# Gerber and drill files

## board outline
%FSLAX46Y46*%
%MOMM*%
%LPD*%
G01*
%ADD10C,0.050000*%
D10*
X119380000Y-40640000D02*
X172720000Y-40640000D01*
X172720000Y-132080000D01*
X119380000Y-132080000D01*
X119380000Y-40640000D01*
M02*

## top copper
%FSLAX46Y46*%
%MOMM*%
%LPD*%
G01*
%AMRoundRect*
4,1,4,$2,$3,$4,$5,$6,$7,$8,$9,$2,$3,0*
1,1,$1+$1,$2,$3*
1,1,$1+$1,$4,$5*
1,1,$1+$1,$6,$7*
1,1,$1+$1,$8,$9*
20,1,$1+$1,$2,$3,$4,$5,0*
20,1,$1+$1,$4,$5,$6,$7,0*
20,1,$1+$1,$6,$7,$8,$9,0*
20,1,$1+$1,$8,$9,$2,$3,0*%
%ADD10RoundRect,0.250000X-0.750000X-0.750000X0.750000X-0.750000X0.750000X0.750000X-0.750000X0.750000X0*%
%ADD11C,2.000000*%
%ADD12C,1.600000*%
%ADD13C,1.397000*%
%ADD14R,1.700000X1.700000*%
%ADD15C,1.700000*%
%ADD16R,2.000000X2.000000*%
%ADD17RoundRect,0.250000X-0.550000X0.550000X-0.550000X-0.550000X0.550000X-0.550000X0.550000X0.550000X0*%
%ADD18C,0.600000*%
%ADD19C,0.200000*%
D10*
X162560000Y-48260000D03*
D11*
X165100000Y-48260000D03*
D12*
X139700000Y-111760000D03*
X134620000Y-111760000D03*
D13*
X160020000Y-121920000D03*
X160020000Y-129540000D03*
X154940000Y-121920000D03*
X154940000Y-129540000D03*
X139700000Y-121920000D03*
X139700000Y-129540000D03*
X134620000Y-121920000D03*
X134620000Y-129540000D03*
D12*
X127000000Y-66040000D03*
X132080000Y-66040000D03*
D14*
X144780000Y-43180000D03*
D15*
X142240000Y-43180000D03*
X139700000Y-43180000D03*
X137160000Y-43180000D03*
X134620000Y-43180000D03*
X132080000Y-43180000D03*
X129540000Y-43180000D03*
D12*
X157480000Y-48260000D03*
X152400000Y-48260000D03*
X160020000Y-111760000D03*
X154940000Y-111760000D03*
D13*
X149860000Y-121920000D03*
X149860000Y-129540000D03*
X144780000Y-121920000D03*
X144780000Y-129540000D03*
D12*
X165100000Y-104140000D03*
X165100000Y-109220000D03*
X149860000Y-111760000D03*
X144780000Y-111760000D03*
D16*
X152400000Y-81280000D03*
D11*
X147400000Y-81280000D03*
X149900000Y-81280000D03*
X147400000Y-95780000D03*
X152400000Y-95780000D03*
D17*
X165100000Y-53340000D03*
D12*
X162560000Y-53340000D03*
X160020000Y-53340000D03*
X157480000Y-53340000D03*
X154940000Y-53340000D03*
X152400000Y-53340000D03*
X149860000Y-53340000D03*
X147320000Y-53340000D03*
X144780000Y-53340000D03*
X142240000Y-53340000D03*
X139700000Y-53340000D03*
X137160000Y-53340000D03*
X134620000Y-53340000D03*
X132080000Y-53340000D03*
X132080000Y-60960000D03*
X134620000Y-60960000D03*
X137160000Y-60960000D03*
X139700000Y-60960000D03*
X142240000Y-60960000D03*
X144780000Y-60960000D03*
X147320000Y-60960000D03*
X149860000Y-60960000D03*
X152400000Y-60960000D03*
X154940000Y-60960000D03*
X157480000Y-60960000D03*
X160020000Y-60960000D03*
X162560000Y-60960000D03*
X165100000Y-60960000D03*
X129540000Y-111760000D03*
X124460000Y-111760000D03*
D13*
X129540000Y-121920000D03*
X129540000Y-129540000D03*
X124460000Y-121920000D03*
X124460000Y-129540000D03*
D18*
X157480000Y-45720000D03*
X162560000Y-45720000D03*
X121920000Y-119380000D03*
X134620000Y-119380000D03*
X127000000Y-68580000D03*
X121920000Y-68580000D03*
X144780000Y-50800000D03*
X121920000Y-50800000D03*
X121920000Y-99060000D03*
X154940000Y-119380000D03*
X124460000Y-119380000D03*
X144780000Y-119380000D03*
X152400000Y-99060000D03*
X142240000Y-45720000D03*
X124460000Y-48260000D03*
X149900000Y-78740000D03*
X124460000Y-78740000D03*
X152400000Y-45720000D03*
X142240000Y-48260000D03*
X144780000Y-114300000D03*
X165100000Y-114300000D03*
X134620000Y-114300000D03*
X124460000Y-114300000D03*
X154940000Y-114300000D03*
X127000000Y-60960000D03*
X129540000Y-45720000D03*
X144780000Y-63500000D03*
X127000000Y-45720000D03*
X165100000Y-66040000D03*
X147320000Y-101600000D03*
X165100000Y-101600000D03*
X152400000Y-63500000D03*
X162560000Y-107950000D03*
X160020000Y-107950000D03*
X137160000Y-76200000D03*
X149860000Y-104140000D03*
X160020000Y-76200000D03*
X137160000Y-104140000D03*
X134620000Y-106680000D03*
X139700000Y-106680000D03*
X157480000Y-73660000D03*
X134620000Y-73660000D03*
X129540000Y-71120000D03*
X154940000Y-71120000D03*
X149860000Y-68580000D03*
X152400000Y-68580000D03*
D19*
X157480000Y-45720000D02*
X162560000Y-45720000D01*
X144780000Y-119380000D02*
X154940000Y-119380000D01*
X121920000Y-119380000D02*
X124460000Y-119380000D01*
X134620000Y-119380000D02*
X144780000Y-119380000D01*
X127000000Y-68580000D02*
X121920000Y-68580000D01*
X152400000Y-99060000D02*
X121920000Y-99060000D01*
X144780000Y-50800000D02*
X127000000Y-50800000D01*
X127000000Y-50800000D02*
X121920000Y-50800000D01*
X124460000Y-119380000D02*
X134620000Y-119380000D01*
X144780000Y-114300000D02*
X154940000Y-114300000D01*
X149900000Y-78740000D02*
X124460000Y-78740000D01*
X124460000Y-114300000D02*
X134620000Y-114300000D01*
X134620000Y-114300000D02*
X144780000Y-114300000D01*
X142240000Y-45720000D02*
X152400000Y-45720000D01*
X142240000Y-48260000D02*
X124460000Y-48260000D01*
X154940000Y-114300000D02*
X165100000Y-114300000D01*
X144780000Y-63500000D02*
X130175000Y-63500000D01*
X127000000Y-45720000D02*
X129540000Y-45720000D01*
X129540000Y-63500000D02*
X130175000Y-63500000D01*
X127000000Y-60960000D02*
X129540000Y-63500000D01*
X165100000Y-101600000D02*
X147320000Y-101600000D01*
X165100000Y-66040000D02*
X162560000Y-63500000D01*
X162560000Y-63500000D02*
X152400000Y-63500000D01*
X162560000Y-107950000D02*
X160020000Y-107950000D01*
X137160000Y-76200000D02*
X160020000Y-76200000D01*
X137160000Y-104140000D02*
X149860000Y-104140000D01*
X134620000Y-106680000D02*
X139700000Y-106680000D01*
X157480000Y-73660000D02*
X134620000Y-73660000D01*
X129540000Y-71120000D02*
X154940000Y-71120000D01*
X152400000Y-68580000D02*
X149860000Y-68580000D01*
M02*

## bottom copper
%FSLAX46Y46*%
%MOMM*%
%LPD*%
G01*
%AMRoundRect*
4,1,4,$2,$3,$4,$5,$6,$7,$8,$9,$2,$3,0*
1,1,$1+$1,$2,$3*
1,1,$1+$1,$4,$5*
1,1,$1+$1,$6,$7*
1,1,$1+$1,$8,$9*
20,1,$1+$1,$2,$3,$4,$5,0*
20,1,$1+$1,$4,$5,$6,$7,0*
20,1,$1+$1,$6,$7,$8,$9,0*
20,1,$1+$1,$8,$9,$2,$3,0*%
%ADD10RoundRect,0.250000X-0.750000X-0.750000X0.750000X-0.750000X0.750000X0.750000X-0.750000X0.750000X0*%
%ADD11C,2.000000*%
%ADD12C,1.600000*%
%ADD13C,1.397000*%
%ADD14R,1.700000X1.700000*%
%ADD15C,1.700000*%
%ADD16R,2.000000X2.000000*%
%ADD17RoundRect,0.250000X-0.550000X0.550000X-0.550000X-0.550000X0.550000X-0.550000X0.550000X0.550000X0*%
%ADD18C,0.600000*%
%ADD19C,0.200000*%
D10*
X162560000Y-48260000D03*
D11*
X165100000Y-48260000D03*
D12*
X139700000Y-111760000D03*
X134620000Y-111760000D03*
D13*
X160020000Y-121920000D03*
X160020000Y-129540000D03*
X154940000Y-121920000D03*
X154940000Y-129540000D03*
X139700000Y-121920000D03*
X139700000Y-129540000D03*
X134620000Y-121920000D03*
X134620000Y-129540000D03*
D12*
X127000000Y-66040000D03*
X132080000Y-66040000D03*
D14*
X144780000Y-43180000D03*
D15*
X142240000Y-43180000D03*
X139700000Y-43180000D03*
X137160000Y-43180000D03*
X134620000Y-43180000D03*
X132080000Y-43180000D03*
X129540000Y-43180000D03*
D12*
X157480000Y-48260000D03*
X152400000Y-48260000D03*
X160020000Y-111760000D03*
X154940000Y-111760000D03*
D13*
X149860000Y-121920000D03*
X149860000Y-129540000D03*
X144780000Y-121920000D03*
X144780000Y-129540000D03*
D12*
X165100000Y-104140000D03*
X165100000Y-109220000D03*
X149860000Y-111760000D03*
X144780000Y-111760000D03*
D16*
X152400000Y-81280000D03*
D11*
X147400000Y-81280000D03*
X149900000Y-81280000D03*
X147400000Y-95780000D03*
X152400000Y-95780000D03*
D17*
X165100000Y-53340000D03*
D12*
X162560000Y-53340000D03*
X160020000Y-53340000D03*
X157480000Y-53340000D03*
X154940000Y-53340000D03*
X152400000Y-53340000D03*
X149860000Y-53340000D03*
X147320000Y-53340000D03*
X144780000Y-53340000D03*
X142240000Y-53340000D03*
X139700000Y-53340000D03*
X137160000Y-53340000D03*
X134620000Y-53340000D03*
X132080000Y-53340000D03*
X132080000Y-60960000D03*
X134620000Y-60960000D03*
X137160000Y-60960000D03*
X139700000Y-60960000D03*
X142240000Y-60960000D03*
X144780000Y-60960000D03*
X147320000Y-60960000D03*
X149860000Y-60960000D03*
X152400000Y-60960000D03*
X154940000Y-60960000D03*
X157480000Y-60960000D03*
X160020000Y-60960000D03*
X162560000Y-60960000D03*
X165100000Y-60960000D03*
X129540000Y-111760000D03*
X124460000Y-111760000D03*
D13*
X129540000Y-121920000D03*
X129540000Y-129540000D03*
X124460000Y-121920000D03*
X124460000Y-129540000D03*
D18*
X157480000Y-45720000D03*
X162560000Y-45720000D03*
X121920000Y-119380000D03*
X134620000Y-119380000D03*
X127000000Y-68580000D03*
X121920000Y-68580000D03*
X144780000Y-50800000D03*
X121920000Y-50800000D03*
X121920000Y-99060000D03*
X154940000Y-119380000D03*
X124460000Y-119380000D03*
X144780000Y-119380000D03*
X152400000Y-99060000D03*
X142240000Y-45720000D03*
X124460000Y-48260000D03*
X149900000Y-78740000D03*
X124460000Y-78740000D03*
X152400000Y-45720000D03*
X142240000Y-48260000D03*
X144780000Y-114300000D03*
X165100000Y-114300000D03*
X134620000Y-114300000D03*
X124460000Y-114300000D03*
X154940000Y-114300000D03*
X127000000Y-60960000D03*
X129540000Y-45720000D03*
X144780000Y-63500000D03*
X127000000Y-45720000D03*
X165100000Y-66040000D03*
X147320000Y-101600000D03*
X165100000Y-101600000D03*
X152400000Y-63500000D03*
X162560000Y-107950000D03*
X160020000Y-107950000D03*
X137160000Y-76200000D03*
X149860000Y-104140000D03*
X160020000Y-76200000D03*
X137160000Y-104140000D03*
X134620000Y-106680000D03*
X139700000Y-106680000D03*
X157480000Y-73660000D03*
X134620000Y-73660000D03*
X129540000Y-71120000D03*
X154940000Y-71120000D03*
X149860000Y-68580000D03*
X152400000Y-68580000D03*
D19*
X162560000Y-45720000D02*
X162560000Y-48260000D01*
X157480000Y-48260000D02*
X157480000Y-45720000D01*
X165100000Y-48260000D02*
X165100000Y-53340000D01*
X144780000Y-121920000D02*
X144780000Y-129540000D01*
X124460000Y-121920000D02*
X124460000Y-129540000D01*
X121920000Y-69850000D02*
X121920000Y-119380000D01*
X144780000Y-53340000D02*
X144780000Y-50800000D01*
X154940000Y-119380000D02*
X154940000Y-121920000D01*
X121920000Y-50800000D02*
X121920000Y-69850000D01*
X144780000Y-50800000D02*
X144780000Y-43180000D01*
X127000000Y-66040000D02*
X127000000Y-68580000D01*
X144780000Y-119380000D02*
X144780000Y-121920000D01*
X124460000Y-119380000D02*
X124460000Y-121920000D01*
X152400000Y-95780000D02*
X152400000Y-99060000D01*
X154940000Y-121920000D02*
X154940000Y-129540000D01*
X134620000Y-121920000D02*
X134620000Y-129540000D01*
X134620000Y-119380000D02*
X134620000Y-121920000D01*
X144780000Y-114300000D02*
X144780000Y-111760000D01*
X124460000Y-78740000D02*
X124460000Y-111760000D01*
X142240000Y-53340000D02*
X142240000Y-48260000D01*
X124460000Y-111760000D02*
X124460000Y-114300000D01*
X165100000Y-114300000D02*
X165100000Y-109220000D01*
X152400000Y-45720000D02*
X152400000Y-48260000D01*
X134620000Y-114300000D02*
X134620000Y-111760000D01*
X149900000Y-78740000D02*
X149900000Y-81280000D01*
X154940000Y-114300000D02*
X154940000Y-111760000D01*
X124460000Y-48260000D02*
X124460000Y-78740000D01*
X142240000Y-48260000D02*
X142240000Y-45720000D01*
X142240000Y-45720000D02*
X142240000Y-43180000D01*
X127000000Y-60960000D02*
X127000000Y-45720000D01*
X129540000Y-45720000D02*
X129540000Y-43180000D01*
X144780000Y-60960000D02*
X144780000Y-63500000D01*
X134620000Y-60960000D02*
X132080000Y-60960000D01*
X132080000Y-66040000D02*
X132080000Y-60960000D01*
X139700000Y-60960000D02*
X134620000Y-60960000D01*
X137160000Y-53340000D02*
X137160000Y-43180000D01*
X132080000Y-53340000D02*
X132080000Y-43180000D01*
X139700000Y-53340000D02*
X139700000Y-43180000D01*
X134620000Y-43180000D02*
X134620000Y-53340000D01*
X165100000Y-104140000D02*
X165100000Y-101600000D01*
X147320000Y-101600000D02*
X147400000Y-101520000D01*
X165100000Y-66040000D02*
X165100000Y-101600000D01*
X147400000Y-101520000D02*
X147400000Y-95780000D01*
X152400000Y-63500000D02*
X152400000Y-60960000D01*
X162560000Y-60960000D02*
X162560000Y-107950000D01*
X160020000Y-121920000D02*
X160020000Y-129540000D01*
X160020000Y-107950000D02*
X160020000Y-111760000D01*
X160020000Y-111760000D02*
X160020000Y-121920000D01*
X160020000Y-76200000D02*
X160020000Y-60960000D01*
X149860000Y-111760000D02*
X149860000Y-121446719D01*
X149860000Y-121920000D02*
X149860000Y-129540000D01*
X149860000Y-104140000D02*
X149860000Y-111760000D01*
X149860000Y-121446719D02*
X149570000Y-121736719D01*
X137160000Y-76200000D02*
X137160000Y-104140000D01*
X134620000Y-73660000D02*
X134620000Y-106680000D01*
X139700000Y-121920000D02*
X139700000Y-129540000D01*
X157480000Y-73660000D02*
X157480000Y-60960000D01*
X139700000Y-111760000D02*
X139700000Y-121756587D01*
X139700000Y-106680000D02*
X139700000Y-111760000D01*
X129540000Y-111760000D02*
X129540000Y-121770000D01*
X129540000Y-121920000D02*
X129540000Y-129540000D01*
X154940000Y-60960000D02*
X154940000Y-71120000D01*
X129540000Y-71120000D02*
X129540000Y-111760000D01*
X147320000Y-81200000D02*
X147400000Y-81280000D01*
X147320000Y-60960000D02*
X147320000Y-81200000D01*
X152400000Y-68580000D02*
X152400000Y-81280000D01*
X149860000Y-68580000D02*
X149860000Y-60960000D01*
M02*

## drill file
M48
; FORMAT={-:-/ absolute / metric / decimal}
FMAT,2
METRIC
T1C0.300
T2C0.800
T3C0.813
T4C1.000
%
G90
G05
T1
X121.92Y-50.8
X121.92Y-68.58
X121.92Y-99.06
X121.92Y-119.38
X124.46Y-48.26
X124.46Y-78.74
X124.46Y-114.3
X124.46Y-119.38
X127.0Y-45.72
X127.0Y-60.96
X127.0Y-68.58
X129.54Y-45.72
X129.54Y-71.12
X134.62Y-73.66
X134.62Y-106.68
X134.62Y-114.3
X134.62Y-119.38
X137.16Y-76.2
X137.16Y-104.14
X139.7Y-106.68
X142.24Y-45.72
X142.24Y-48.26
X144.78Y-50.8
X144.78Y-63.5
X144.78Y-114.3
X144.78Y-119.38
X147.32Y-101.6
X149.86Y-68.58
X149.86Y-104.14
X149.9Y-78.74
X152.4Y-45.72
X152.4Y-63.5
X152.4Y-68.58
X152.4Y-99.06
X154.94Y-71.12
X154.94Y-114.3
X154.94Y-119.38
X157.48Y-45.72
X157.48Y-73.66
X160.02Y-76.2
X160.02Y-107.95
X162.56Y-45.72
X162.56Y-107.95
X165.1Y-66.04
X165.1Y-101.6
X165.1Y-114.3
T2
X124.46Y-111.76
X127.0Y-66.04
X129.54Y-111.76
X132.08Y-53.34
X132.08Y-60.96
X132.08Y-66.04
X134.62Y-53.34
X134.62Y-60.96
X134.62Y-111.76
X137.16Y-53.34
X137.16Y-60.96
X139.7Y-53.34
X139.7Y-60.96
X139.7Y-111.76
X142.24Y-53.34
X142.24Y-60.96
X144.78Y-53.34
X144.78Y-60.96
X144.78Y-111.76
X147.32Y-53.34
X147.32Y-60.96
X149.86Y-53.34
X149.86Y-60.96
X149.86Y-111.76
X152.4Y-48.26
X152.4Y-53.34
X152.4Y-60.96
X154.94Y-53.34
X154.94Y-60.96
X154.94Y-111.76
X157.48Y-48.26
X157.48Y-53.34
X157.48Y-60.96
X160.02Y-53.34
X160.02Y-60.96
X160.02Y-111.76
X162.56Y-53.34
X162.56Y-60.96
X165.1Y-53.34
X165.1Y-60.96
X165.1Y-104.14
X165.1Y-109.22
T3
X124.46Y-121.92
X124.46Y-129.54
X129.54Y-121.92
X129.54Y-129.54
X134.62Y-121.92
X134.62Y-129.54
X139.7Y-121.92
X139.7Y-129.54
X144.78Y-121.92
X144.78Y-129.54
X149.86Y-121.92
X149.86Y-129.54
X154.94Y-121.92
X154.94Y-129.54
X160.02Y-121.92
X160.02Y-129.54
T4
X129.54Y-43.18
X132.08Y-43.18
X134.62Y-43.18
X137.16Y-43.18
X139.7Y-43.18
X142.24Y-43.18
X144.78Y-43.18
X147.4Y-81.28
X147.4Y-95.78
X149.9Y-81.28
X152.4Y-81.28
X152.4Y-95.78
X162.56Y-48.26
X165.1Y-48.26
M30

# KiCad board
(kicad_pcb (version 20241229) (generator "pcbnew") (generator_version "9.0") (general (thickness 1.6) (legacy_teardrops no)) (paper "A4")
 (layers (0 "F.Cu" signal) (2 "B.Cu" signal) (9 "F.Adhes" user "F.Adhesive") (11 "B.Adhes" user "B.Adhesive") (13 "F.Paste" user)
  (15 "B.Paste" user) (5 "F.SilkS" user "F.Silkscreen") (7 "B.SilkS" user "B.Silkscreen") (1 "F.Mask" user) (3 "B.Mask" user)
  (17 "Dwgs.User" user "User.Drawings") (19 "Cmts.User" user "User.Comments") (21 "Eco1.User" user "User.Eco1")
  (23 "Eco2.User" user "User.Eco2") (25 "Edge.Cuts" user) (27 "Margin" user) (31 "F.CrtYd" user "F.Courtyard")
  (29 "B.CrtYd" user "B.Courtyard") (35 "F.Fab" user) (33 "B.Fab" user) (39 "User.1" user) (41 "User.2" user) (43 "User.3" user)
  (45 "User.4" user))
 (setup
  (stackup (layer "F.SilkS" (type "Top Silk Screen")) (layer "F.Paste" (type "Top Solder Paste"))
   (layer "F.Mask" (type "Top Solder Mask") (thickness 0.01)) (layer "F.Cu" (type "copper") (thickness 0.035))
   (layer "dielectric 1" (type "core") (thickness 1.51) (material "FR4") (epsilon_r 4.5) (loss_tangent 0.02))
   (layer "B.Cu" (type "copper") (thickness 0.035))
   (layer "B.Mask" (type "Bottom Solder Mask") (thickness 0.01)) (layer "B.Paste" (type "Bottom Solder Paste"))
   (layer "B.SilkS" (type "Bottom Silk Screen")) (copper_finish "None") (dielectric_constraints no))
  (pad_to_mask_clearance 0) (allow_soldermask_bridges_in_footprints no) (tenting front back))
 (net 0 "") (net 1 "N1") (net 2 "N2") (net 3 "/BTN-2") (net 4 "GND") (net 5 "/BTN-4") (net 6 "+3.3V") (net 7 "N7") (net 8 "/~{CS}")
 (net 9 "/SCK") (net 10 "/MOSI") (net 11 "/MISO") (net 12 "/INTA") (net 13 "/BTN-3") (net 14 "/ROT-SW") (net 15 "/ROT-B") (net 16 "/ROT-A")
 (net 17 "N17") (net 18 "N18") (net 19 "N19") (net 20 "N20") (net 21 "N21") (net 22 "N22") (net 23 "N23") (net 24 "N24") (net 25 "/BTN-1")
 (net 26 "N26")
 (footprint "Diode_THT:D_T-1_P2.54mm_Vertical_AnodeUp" (layer "F.Cu") (at 162.56 48.26)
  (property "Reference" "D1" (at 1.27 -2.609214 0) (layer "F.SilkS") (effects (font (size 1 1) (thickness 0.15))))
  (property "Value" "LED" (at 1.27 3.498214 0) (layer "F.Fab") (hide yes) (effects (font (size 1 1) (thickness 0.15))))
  (pad "1" thru_hole roundrect (at 0 0) (size 2 2) (drill 1) (layers "*.Cu" "*.Mask") (remove_unused_layers no) (roundrect_rratio 0.125)
   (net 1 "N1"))
  (pad "2" thru_hole circle (at 2.54 0) (size 2 2) (drill 1) (layers "*.Cu" "*.Mask") (remove_unused_layers no) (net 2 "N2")))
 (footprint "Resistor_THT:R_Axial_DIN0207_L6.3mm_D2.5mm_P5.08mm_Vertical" (layer "F.Cu") (at 139.7 111.76 180)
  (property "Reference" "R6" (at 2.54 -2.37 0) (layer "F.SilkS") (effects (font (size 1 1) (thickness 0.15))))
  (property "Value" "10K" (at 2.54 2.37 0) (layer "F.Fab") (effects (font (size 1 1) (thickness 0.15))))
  (pad "1" thru_hole circle (at 0 0 180) (size 1.6 1.6) (drill 0.8) (layers "*.Cu" "*.Mask") (remove_unused_layers no) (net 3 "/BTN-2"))
  (pad "2" thru_hole circle (at 5.08 0 180) (size 1.6 1.6) (drill 0.8) (layers "*.Cu" "*.Mask") (remove_unused_layers no) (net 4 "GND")))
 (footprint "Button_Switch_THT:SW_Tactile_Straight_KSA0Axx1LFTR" (layer "F.Cu") (at 160.02 121.92 -90)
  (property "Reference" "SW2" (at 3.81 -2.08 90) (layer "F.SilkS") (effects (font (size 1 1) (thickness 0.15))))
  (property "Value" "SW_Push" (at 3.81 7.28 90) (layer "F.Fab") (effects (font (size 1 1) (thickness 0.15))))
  (pad "1" thru_hole circle (at 0 0 270) (size 1.397 1.397) (drill 0.8128) (layers "*.Cu" "*.Mask") (remove_unused_layers no)
   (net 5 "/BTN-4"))
  (pad "1" thru_hole circle (at 7.62 0 270) (size 1.397 1.397) (drill 0.8128) (layers "*.Cu" "*.Mask") (remove_unused_layers no)
   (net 5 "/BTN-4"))
  (pad "2" thru_hole circle (at 0 5.08 270) (size 1.397 1.397) (drill 0.8128) (layers "*.Cu" "*.Mask") (remove_unused_layers no)
   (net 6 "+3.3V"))
  (pad "2" thru_hole circle (at 7.62 5.08 270) (size 1.397 1.397) (drill 0.8128) (layers "*.Cu" "*.Mask") (remove_unused_layers no)
   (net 6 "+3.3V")))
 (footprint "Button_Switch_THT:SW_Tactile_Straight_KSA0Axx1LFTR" (layer "F.Cu") (at 139.7 121.92 -90)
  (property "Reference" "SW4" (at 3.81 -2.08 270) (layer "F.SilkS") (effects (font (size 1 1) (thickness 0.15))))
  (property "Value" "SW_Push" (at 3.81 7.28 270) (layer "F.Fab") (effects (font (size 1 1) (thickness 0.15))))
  (pad "1" thru_hole circle (at 0 0 270) (size 1.397 1.397) (drill 0.8128) (layers "*.Cu" "*.Mask") (remove_unused_layers no)
   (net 3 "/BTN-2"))
  (pad "1" thru_hole circle (at 7.62 0 270) (size 1.397 1.397) (drill 0.8128) (layers "*.Cu" "*.Mask") (remove_unused_layers no)
   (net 3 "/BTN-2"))
  (pad "2" thru_hole circle (at 0 5.08 270) (size 1.397 1.397) (drill 0.8128) (layers "*.Cu" "*.Mask") (remove_unused_layers no)
   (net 6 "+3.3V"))
  (pad "2" thru_hole circle (at 7.62 5.08 270) (size 1.397 1.397) (drill 0.8128) (layers "*.Cu" "*.Mask") (remove_unused_layers no)
   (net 6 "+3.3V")))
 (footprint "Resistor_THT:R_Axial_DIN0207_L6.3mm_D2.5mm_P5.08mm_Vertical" (layer "F.Cu") (at 127 66.04)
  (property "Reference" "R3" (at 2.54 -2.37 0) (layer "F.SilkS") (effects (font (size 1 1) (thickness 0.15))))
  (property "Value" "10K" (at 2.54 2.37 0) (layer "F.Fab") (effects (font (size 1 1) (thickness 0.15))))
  (pad "1" thru_hole circle (at 0 0) (size 1.6 1.6) (drill 0.8) (layers "*.Cu" "*.Mask") (remove_unused_layers no) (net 6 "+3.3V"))
  (pad "2" thru_hole circle (at 5.08 0) (size 1.6 1.6) (drill 0.8) (layers "*.Cu" "*.Mask") (remove_unused_layers no) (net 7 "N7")))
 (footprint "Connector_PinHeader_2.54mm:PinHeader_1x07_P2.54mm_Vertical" (layer "F.Cu") (at 144.78 43.18 -90)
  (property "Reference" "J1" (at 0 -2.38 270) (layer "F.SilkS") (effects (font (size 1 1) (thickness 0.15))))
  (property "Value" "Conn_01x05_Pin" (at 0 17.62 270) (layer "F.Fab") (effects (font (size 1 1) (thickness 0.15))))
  (pad "1" thru_hole rect (at 0 0 270) (size 1.7 1.7) (drill 1) (layers "*.Cu" "*.Mask") (remove_unused_layers no) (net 6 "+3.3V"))
  (pad "2" thru_hole circle (at 0 2.54 270) (size 1.7 1.7) (drill 1) (layers "*.Cu" "*.Mask") (remove_unused_layers no) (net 4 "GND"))
  (pad "3" thru_hole circle (at 0 5.08 270) (size 1.7 1.7) (drill 1) (layers "*.Cu" "*.Mask") (remove_unused_layers no) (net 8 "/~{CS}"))
  (pad "4" thru_hole circle (at 0 7.62 270) (size 1.7 1.7) (drill 1) (layers "*.Cu" "*.Mask") (remove_unused_layers no) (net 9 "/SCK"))
  (pad "5" thru_hole circle (at 0 10.16 270) (size 1.7 1.7) (drill 1) (layers "*.Cu" "*.Mask") (remove_unused_layers no) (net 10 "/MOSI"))
  (pad "6" thru_hole circle (at 0 12.7 270) (size 1.7 1.7) (drill 1) (layers "*.Cu" "*.Mask") (remove_unused_layers no) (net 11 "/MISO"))
  (pad "7" thru_hole circle (at 0 15.24 270) (size 1.7 1.7) (drill 1) (layers "*.Cu" "*.Mask") (remove_unused_layers no) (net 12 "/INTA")))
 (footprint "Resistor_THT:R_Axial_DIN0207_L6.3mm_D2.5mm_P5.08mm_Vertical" (layer "F.Cu") (at 157.48 48.26 180)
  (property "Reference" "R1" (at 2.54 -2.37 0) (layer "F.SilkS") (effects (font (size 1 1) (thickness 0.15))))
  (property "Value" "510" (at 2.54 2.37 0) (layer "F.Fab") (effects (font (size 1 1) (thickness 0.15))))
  (pad "1" thru_hole circle (at 0 0 180) (size 1.6 1.6) (drill 0.8) (layers "*.Cu" "*.Mask") (remove_unused_layers no) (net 1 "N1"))
  (pad "2" thru_hole circle (at 5.08 0 180) (size 1.6 1.6) (drill 0.8) (layers "*.Cu" "*.Mask") (remove_unused_layers no) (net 4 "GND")))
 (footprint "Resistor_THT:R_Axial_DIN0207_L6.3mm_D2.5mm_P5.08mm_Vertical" (layer "F.Cu") (at 160.02 111.76 180)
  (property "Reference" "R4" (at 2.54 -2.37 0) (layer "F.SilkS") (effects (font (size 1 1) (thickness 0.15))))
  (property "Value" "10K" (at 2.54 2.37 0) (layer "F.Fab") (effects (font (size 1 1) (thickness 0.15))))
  (pad "1" thru_hole circle (at 0 0 180) (size 1.6 1.6) (drill 0.8) (layers "*.Cu" "*.Mask") (remove_unused_layers no) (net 5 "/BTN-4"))
  (pad "2" thru_hole circle (at 5.08 0 180) (size 1.6 1.6) (drill 0.8) (layers "*.Cu" "*.Mask") (remove_unused_layers no) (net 4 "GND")))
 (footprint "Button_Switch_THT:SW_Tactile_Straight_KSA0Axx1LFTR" (layer "F.Cu") (at 149.86 121.92 -90)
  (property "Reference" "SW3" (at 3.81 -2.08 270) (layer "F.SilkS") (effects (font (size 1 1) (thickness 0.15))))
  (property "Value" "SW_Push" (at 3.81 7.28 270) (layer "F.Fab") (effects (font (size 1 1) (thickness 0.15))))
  (pad "1" thru_hole circle (at 0 0 270) (size 1.397 1.397) (drill 0.8128) (layers "*.Cu" "*.Mask") (remove_unused_layers no)
   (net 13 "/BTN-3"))
  (pad "1" thru_hole circle (at 7.62 0 270) (size 1.397 1.397) (drill 0.8128) (layers "*.Cu" "*.Mask") (remove_unused_layers no)
   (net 13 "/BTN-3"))
  (pad "2" thru_hole circle (at 0 5.08 270) (size 1.397 1.397) (drill 0.8128) (layers "*.Cu" "*.Mask") (remove_unused_layers no)
   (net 6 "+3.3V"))
  (pad "2" thru_hole circle (at 7.62 5.08 270) (size 1.397 1.397) (drill 0.8128) (layers "*.Cu" "*.Mask") (remove_unused_layers no)
   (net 6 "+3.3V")))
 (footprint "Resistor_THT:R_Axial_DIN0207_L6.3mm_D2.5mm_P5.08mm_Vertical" (layer "F.Cu") (at 165.1 104.14 -90)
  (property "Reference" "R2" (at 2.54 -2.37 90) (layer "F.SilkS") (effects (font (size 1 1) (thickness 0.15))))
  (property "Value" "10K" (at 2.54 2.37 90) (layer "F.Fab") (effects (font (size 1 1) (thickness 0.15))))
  (pad "1" thru_hole circle (at 0 0 270) (size 1.6 1.6) (drill 0.8) (layers "*.Cu" "*.Mask") (remove_unused_layers no) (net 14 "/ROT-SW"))
  (pad "2" thru_hole circle (at 5.08 0 270) (size 1.6 1.6) (drill 0.8) (layers "*.Cu" "*.Mask") (remove_unused_layers no) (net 4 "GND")))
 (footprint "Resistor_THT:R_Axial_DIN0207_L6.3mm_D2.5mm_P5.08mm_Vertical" (layer "F.Cu") (at 149.86 111.76 180)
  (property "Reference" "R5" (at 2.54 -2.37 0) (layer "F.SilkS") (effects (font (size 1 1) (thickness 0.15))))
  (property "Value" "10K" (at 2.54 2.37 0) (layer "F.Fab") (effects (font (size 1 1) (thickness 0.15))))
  (pad "1" thru_hole circle (at 0 0 180) (size 1.6 1.6) (drill 0.8) (layers "*.Cu" "*.Mask") (remove_unused_layers no) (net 13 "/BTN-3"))
  (pad "2" thru_hole circle (at 5.08 0 180) (size 1.6 1.6) (drill 0.8) (layers "*.Cu" "*.Mask") (remove_unused_layers no) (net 4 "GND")))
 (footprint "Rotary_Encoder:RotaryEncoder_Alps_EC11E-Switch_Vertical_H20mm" (layer "F.Cu") (at 152.4 81.28 -90)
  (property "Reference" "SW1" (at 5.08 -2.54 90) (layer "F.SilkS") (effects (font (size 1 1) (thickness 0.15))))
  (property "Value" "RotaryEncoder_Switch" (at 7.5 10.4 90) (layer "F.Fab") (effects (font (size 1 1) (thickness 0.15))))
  (pad "A" thru_hole rect (at 0 0 270) (size 2 2) (drill 1) (layers "*.Cu" "*.Mask") (remove_unused_layers no) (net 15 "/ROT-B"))
  (pad "B" thru_hole circle (at 0 5 270) (size 2 2) (drill 1) (layers "*.Cu" "*.Mask") (remove_unused_layers no) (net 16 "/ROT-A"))
  (pad "C" thru_hole circle (at 0 2.5 270) (size 2 2) (drill 1) (layers "*.Cu" "*.Mask") (remove_unused_layers no) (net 4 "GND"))
  (pad "S1" thru_hole circle (at 14.5 5 270) (size 2 2) (drill 1) (layers "*.Cu" "*.Mask") (remove_unused_layers no) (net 14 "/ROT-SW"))
  (pad "S2" thru_hole circle (at 14.5 0 270) (size 2 2) (drill 1) (layers "*.Cu" "*.Mask") (remove_unused_layers no) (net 6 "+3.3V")))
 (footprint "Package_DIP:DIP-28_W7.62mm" (layer "F.Cu") (at 165.1 53.34 -90)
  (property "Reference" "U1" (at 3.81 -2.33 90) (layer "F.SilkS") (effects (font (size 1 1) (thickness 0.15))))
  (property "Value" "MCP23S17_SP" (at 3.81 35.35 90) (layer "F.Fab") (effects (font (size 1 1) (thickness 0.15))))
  (pad "1" thru_hole roundrect (at 0 0 270) (size 1.6 1.6) (drill 0.8) (layers "*.Cu" "*.Mask") (remove_unused_layers no)
   (roundrect_rratio 0.15625) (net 2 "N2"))
  (pad "2" thru_hole circle (at 0 2.54 270) (size 1.6 1.6) (drill 0.8) (layers "*.Cu" "*.Mask") (remove_unused_layers no) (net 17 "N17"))
  (pad "3" thru_hole circle (at 0 5.08 270) (size 1.6 1.6) (drill 0.8) (layers "*.Cu" "*.Mask") (remove_unused_layers no) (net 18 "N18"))
  (pad "4" thru_hole circle (at 0 7.62 270) (size 1.6 1.6) (drill 0.8) (layers "*.Cu" "*.Mask") (remove_unused_layers no) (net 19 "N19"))
  (pad "5" thru_hole circle (at 0 10.16 270) (size 1.6 1.6) (drill 0.8) (layers "*.Cu" "*.Mask") (remove_unused_layers no) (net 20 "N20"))
  (pad "6" thru_hole circle (at 0 12.7 270) (size 1.6 1.6) (drill 0.8) (layers "*.Cu" "*.Mask") (remove_unused_layers no) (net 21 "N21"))
  (pad "7" thru_hole circle (at 0 15.24 270) (size 1.6 1.6) (drill 0.8) (layers "*.Cu" "*.Mask") (remove_unused_layers no) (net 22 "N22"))
  (pad "8" thru_hole circle (at 0 17.78 270) (size 1.6 1.6) (drill 0.8) (layers "*.Cu" "*.Mask") (remove_unused_layers no) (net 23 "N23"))
  (pad "9" thru_hole circle (at 0 20.32 270) (size 1.6 1.6) (drill 0.8) (layers "*.Cu" "*.Mask") (remove_unused_layers no) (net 6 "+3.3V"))
  (pad "10" thru_hole circle (at 0 22.86 270) (size 1.6 1.6) (drill 0.8) (layers "*.Cu" "*.Mask") (remove_unused_layers no) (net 4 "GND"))
  (pad "11" thru_hole circle (at 0 25.4 270) (size 1.6 1.6) (drill 0.8) (layers "*.Cu" "*.Mask") (remove_unused_layers no) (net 8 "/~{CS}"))
  (pad "12" thru_hole circle (at 0 27.94 270) (size 1.6 1.6) (drill 0.8) (layers "*.Cu" "*.Mask") (remove_unused_layers no) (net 9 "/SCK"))
  (pad "13" thru_hole circle (at 0 30.48 270) (size 1.6 1.6) (drill 0.8) (layers "*.Cu" "*.Mask") (remove_unused_layers no) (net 10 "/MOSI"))
  (pad "14" thru_hole circle (at 0 33.02 270) (size 1.6 1.6) (drill 0.8) (layers "*.Cu" "*.Mask") (remove_unused_layers no) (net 11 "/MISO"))
  (pad "15" thru_hole circle (at 7.62 33.02 270) (size 1.6 1.6) (drill 0.8) (layers "*.Cu" "*.Mask") (remove_unused_layers no) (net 7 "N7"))
  (pad "16" thru_hole circle (at 7.62 30.48 270) (size 1.6 1.6) (drill 0.8) (layers "*.Cu" "*.Mask") (remove_unused_layers no) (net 7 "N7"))
  (pad "17" thru_hole circle (at 7.62 27.94 270) (size 1.6 1.6) (drill 0.8) (layers "*.Cu" "*.Mask") (remove_unused_layers no) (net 7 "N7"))
  (pad "18" thru_hole circle (at 7.62 25.4 270) (size 1.6 1.6) (drill 0.8) (layers "*.Cu" "*.Mask") (remove_unused_layers no) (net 7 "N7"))
  (pad "19" thru_hole circle (at 7.62 22.86 270) (size 1.6 1.6) (drill 0.8) (layers "*.Cu" "*.Mask") (remove_unused_layers no)
   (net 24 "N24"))
  (pad "20" thru_hole circle (at 7.62 20.32 270) (size 1.6 1.6) (drill 0.8) (layers "*.Cu" "*.Mask") (remove_unused_layers no)
   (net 12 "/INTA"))
  (pad "21" thru_hole circle (at 7.62 17.78 270) (size 1.6 1.6) (drill 0.8) (layers "*.Cu" "*.Mask") (remove_unused_layers no)
   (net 16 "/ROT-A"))
  (pad "22" thru_hole circle (at 7.62 15.24 270) (size 1.6 1.6) (drill 0.8) (layers "*.Cu" "*.Mask") (remove_unused_layers no)
   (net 15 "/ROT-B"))
  (pad "23" thru_hole circle (at 7.62 12.7 270) (size 1.6 1.6) (drill 0.8) (layers "*.Cu" "*.Mask") (remove_unused_layers no)
   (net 14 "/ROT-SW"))
  (pad "24" thru_hole circle (at 7.62 10.16 270) (size 1.6 1.6) (drill 0.8) (layers "*.Cu" "*.Mask") (remove_unused_layers no)
   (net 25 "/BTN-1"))
  (pad "25" thru_hole circle (at 7.62 7.62 270) (size 1.6 1.6) (drill 0.8) (layers "*.Cu" "*.Mask") (remove_unused_layers no)
   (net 3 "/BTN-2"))
  (pad "26" thru_hole circle (at 7.62 5.08 270) (size 1.6 1.6) (drill 0.8) (layers "*.Cu" "*.Mask") (remove_unused_layers no)
   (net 13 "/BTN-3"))
  (pad "27" thru_hole circle (at 7.62 2.54 270) (size 1.6 1.6) (drill 0.8) (layers "*.Cu" "*.Mask") (remove_unused_layers no)
   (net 5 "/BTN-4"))
  (pad "28" thru_hole circle (at 7.62 0 270) (size 1.6 1.6) (drill 0.8) (layers "*.Cu" "*.Mask") (remove_unused_layers no) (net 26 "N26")))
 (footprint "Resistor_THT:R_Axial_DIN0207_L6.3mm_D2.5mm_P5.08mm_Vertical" (layer "F.Cu") (at 129.54 111.76 180)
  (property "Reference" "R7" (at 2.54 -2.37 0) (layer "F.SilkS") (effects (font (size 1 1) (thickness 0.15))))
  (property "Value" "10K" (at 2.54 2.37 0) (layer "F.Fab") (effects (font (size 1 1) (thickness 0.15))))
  (pad "1" thru_hole circle (at 0 0 180) (size 1.6 1.6) (drill 0.8) (layers "*.Cu" "*.Mask") (remove_unused_layers no) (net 25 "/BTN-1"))
  (pad "2" thru_hole circle (at 5.08 0 180) (size 1.6 1.6) (drill 0.8) (layers "*.Cu" "*.Mask") (remove_unused_layers no) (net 4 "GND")))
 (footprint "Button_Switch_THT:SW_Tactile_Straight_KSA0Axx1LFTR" (layer "F.Cu") (at 129.54 121.92 -90)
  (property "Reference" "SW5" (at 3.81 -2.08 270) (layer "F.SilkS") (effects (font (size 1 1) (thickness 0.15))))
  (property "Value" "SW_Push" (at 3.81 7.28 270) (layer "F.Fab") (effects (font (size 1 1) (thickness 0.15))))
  (pad "1" thru_hole circle (at 0 0 270) (size 1.397 1.397) (drill 0.8128) (layers "*.Cu" "*.Mask") (remove_unused_layers no)
   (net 25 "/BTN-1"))
  (pad "1" thru_hole circle (at 7.62 0 270) (size 1.397 1.397) (drill 0.8128) (layers "*.Cu" "*.Mask") (remove_unused_layers no)
   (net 25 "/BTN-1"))
  (pad "2" thru_hole circle (at 0 5.08 270) (size 1.397 1.397) (drill 0.8128) (layers "*.Cu" "*.Mask") (remove_unused_layers no)
   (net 6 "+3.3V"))
  (pad "2" thru_hole circle (at 7.62 5.08 270) (size 1.397 1.397) (drill 0.8128) (layers "*.Cu" "*.Mask") (remove_unused_layers no)
   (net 6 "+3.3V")))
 (gr_rect (start 119.38 40.64) (end 172.72 132.08) (stroke (width 0.05) (type default)) (fill no) (layer "Edge.Cuts"))
 (segment (start 157.48 45.72) (end 162.56 45.72) (width 0.2) (layer "F.Cu") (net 1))
 (via (at 157.48 45.72) (size 0.6) (drill 0.3) (layers "F.Cu" "B.Cu") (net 1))
 (via (at 162.56 45.72) (size 0.6) (drill 0.3) (layers "F.Cu" "B.Cu") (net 1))
 (segment (start 162.56 45.72) (end 162.56 48.26) (width 0.2) (layer "B.Cu") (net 1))
 (segment (start 157.48 48.26) (end 157.48 45.72) (width 0.2) (layer "B.Cu") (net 1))
 (segment (start 165.1 48.26) (end 165.1 53.34) (width 0.2) (layer "B.Cu") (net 2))
 (segment (start 144.78 119.38) (end 154.94 119.38) (width 0.2) (layer "F.Cu") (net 6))
 (segment (start 121.92 119.38) (end 124.46 119.38) (width 0.2) (layer "F.Cu") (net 6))
 (segment (start 134.62 119.38) (end 144.78 119.38) (width 0.2) (layer "F.Cu") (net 6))
 (segment (start 127 68.58) (end 121.92 68.58) (width 0.2) (layer "F.Cu") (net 6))
 (segment (start 152.4 99.06) (end 121.92 99.06) (width 0.2) (layer "F.Cu") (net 6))
 (segment (start 144.78 50.8) (end 127 50.8) (width 0.2) (layer "F.Cu") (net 6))
 (segment (start 127 50.8) (end 121.92 50.8) (width 0.2) (layer "F.Cu") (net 6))
 (segment (start 124.46 119.38) (end 134.62 119.38) (width 0.2) (layer "F.Cu") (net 6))
 (via (at 121.92 119.38) (size 0.6) (drill 0.3) (layers "F.Cu" "B.Cu") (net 6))
 (via (at 134.62 119.38) (size 0.6) (drill 0.3) (layers "F.Cu" "B.Cu") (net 6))
 (via (at 127 68.58) (size 0.6) (drill 0.3) (layers "F.Cu" "B.Cu") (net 6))
 (via (at 121.92 68.58) (size 0.6) (drill 0.3) (layers "F.Cu" "B.Cu") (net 6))
 (via (at 144.78 50.8) (size 0.6) (drill 0.3) (layers "F.Cu" "B.Cu") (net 6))
 (via (at 121.92 50.8) (size 0.6) (drill 0.3) (layers "F.Cu" "B.Cu") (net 6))
 (via (at 121.92 99.06) (size 0.6) (drill 0.3) (layers "F.Cu" "B.Cu") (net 6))
 (via (at 154.94 119.38) (size 0.6) (drill 0.3) (layers "F.Cu" "B.Cu") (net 6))
 (via (at 124.46 119.38) (size 0.6) (drill 0.3) (layers "F.Cu" "B.Cu") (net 6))
 (via (at 144.78 119.38) (size 0.6) (drill 0.3) (layers "F.Cu" "B.Cu") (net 6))
 (via (at 152.4 99.06) (size 0.6) (drill 0.3) (layers "F.Cu" "B.Cu") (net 6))
 (segment (start 144.78 121.92) (end 144.78 129.54) (width 0.2) (layer "B.Cu") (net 6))
 (segment (start 124.46 121.92) (end 124.46 129.54) (width 0.2) (layer "B.Cu") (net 6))
 (segment (start 121.92 69.85) (end 121.92 119.38) (width 0.2) (layer "B.Cu") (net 6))
 (segment (start 144.78 53.34) (end 144.78 50.8) (width 0.2) (layer "B.Cu") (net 6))
 (segment (start 154.94 119.38) (end 154.94 121.92) (width 0.2) (layer "B.Cu") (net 6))
 (segment (start 121.92 50.8) (end 121.92 69.85) (width 0.2) (layer "B.Cu") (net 6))
 (segment (start 144.78 50.8) (end 144.78 43.18) (width 0.2) (layer "B.Cu") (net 6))
 (segment (start 127 66.04) (end 127 68.58) (width 0.2) (layer "B.Cu") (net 6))
 (segment (start 144.78 119.38) (end 144.78 121.92) (width 0.2) (layer "B.Cu") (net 6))
 (segment (start 124.46 119.38) (end 124.46 121.92) (width 0.2) (layer "B.Cu") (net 6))
 (segment (start 152.4 95.78) (end 152.4 99.06) (width 0.2) (layer "B.Cu") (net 6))
 (segment (start 154.94 121.92) (end 154.94 129.54) (width 0.2) (layer "B.Cu") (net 6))
 (segment (start 134.62 121.92) (end 134.62 129.54) (width 0.2) (layer "B.Cu") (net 6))
 (segment (start 134.62 119.38) (end 134.62 121.92) (width 0.2) (layer "B.Cu") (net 6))
 (segment (start 144.78 114.3) (end 154.94 114.3) (width 0.2) (layer "F.Cu") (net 4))
 (segment (start 149.9 78.74) (end 124.46 78.74) (width 0.2) (layer "F.Cu") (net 4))
 (segment (start 124.46 114.3) (end 134.62 114.3) (width 0.2) (layer "F.Cu") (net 4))
 (segment (start 134.62 114.3) (end 144.78 114.3) (width 0.2) (layer "F.Cu") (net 4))
 (segment (start 142.24 45.72) (end 152.4 45.72) (width 0.2) (layer "F.Cu") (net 4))
 (segment (start 142.24 48.26) (end 124.46 48.26) (width 0.2) (layer "F.Cu") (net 4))
 (segment (start 154.94 114.3) (end 165.1 114.3) (width 0.2) (layer "F.Cu") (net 4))
 (via (at 142.24 45.72) (size 0.6) (drill 0.3) (layers "F.Cu" "B.Cu") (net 4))
 (via (at 124.46 48.26) (size 0.6) (drill 0.3) (layers "F.Cu" "B.Cu") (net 4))
 (via (at 149.9 78.74) (size 0.6) (drill 0.3) (layers "F.Cu" "B.Cu") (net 4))
 (via (at 124.46 78.74) (size 0.6) (drill 0.3) (layers "F.Cu" "B.Cu") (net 4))
 (via (at 152.4 45.72) (size 0.6) (drill 0.3) (layers "F.Cu" "B.Cu") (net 4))
 (via (at 142.24 48.26) (size 0.6) (drill 0.3) (layers "F.Cu" "B.Cu") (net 4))
 (via (at 144.78 114.3) (size 0.6) (drill 0.3) (layers "F.Cu" "B.Cu") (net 4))
 (via (at 165.1 114.3) (size 0.6) (drill 0.3) (layers "F.Cu" "B.Cu") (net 4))
 (via (at 134.62 114.3) (size 0.6) (drill 0.3) (layers "F.Cu" "B.Cu") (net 4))
 (via (at 124.46 114.3) (size 0.6) (drill 0.3) (layers "F.Cu" "B.Cu") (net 4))
 (via (at 154.94 114.3) (size 0.6) (drill 0.3) (layers "F.Cu" "B.Cu") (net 4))
 (segment (start 144.78 114.3) (end 144.78 111.76) (width 0.2) (layer "B.Cu") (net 4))
 (segment (start 124.46 78.74) (end 124.46 111.76) (width 0.2) (layer "B.Cu") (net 4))
 (segment (start 142.24 53.34) (end 142.24 48.26) (width 0.2) (layer "B.Cu") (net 4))
 (segment (start 124.46 111.76) (end 124.46 114.3) (width 0.2) (layer "B.Cu") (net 4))
 (segment (start 165.1 114.3) (end 165.1 109.22) (width 0.2) (layer "B.Cu") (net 4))
 (segment (start 152.4 45.72) (end 152.4 48.26) (width 0.2) (layer "B.Cu") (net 4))
 (segment (start 134.62 114.3) (end 134.62 111.76) (width 0.2) (layer "B.Cu") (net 4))
 (segment (start 149.9 78.74) (end 149.9 81.28) (width 0.2) (layer "B.Cu") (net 4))
 (segment (start 154.94 114.3) (end 154.94 111.76) (width 0.2) (layer "B.Cu") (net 4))
 (segment (start 124.46 48.26) (end 124.46 78.74) (width 0.2) (layer "B.Cu") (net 4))
 (segment (start 142.24 48.26) (end 142.24 45.72) (width 0.2) (layer "B.Cu") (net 4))
 (segment (start 142.24 45.72) (end 142.24 43.18) (width 0.2) (layer "B.Cu") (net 4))
 (segment (start 144.78 63.5) (end 130.175 63.5) (width 0.2) (layer "F.Cu") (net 12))
 (segment (start 127 45.72) (end 129.54 45.72) (width 0.2) (layer "F.Cu") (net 12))
 (segment (start 129.54 63.5) (end 130.175 63.5) (width 0.2) (layer "F.Cu") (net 12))
 (segment (start 127 60.96) (end 129.54 63.5) (width 0.2) (layer "F.Cu") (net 12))
 (via (at 127 60.96) (size 0.6) (drill 0.3) (layers "F.Cu" "B.Cu") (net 12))
 (via (at 129.54 45.72) (size 0.6) (drill 0.3) (layers "F.Cu" "B.Cu") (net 12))
 (via (at 144.78 63.5) (size 0.6) (drill 0.3) (layers "F.Cu" "B.Cu") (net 12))
 (via (at 127 45.72) (size 0.6) (drill 0.3) (layers "F.Cu" "B.Cu") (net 12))
 (segment (start 127 60.96) (end 127 45.72) (width 0.2) (layer "B.Cu") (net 12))
 (segment (start 129.54 45.72) (end 129.54 43.18) (width 0.2) (layer "B.Cu") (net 12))
 (segment (start 144.78 60.96) (end 144.78 63.5) (width 0.2) (layer "B.Cu") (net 12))
 (segment (start 134.62 60.96) (end 132.08 60.96) (width 0.2) (layer "B.Cu") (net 7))
 (segment (start 132.08 66.04) (end 132.08 60.96) (width 0.2) (layer "B.Cu") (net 7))
 (segment (start 139.7 60.96) (end 134.62 60.96) (width 0.2) (layer "B.Cu") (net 7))
 (segment (start 137.16 53.34) (end 137.16 43.18) (width 0.2) (layer "B.Cu") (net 9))
 (segment (start 132.08 53.34) (end 132.08 43.18) (width 0.2) (layer "B.Cu") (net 11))
 (segment (start 139.7 53.34) (end 139.7 43.18) (width 0.2) (layer "B.Cu") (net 8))
 (segment (start 134.62 43.18) (end 134.62 53.34) (width 0.2) (layer "B.Cu") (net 10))
 (segment (start 165.1 101.6) (end 147.32 101.6) (width 0.2) (layer "F.Cu") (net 14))
 (segment (start 165.1 66.04) (end 162.56 63.5) (width 0.2) (layer "F.Cu") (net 14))
 (segment (start 162.56 63.5) (end 152.4 63.5) (width 0.2) (layer "F.Cu") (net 14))
 (via (at 165.1 66.04) (size 0.6) (drill 0.3) (layers "F.Cu" "B.Cu") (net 14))
 (via (at 147.32 101.6) (size 0.6) (drill 0.3) (layers "F.Cu" "B.Cu") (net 14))
 (via (at 165.1 101.6) (size 0.6) (drill 0.3) (layers "F.Cu" "B.Cu") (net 14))
 (via (at 152.4 63.5) (size 0.6) (drill 0.3) (layers "F.Cu" "B.Cu") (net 14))
 (segment (start 165.1 104.14) (end 165.1 101.6) (width 0.2) (layer "B.Cu") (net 14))
 (segment (start 147.32 101.6) (end 147.4 101.52) (width 0.2) (layer "B.Cu") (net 14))
 (segment (start 165.1 66.04) (end 165.1 101.6) (width 0.2) (layer "B.Cu") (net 14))
 (segment (start 147.4 101.52) (end 147.4 95.78) (width 0.2) (layer "B.Cu") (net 14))
 (segment (start 152.4 63.5) (end 152.4 60.96) (width 0.2) (layer "B.Cu") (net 14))
 (segment (start 162.56 107.95) (end 160.02 107.95) (width 0.2) (layer "F.Cu") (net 5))
 (via (at 162.56 107.95) (size 0.6) (drill 0.3) (layers "F.Cu" "B.Cu") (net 5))
 (via (at 160.02 107.95) (size 0.6) (drill 0.3) (layers "F.Cu" "B.Cu") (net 5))
 (segment (start 162.56 60.96) (end 162.56 107.95) (width 0.2) (layer "B.Cu") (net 5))
 (segment (start 160.02 121.92) (end 160.02 129.54) (width 0.2) (layer "B.Cu") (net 5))
 (segment (start 160.02 107.95) (end 160.02 111.76) (width 0.2) (layer "B.Cu") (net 5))
 (segment (start 160.02 111.76) (end 160.02 121.92) (width 0.2) (layer "B.Cu") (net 5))
 (segment (start 137.16 76.2) (end 160.02 76.2) (width 0.2) (layer "F.Cu") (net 13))
 (segment (start 137.16 104.14) (end 149.86 104.14) (width 0.2) (layer "F.Cu") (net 13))
 (via (at 137.16 76.2) (size 0.6) (drill 0.3) (layers "F.Cu" "B.Cu") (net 13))
 (via (at 149.86 104.14) (size 0.6) (drill 0.3) (layers "F.Cu" "B.Cu") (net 13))
 (via (at 160.02 76.2) (size 0.6) (drill 0.3) (layers "F.Cu" "B.Cu") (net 13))
 (via (at 137.16 104.14) (size 0.6) (drill 0.3) (layers "F.Cu" "B.Cu") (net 13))
 (segment (start 160.02 76.2) (end 160.02 60.96) (width 0.2) (layer "B.Cu") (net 13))
 (segment (start 149.86 111.76) (end 149.86 121.446719) (width 0.2) (layer "B.Cu") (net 13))
 (segment (start 149.86 121.92) (end 149.86 129.54) (width 0.2) (layer "B.Cu") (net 13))
 (segment (start 149.86 104.14) (end 149.86 111.76) (width 0.2) (layer "B.Cu") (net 13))
 (segment (start 149.86 121.446719) (end 149.57 121.736719) (width 0.2) (layer "B.Cu") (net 13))
 (segment (start 137.16 76.2) (end 137.16 104.14) (width 0.2) (layer "B.Cu") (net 13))
 (segment (start 134.62 106.68) (end 139.7 106.68) (width 0.2) (layer "F.Cu") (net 3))
 (segment (start 157.48 73.66) (end 134.62 73.66) (width 0.2) (layer "F.Cu") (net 3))
 (via (at 134.62 106.68) (size 0.6) (drill 0.3) (layers "F.Cu" "B.Cu") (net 3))
 (via (at 139.7 106.68) (size 0.6) (drill 0.3) (layers "F.Cu" "B.Cu") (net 3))
 (via (at 157.48 73.66) (size 0.6) (drill 0.3) (layers "F.Cu" "B.Cu") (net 3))
 (via (at 134.62 73.66) (size 0.6) (drill 0.3) (layers "F.Cu" "B.Cu") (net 3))
 (segment (start 134.62 73.66) (end 134.62 106.68) (width 0.2) (layer "B.Cu") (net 3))
 (segment (start 139.7 121.92) (end 139.7 129.54) (width 0.2) (layer "B.Cu") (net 3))
 (segment (start 157.48 73.66) (end 157.48 60.96) (width 0.2) (layer "B.Cu") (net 3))
 (segment (start 139.7 111.76) (end 139.7 121.756587) (width 0.2) (layer "B.Cu") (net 3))
 (segment (start 139.7 106.68) (end 139.7 111.76) (width 0.2) (layer "B.Cu") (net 3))
 (segment (start 129.54 71.12) (end 154.94 71.12) (width 0.2) (layer "F.Cu") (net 25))
 (via (at 129.54 71.12) (size 0.6) (drill 0.3) (layers "F.Cu" "B.Cu") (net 25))
 (via (at 154.94 71.12) (size 0.6) (drill 0.3) (layers "F.Cu" "B.Cu") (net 25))
 (segment (start 129.54 111.76) (end 129.54 121.77) (width 0.2) (layer "B.Cu") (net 25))
 (segment (start 129.54 121.92) (end 129.54 129.54) (width 0.2) (layer "B.Cu") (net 25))
 (segment (start 154.94 60.96) (end 154.94 71.12) (width 0.2) (layer "B.Cu") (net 25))
 (segment (start 129.54 71.12) (end 129.54 111.76) (width 0.2) (layer "B.Cu") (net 25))
 (segment (start 147.32 81.2) (end 147.4 81.28) (width 0.2) (layer "B.Cu") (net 16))
 (segment (start 147.32 60.96) (end 147.32 81.2) (width 0.2) (layer "B.Cu") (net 16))
 (segment (start 152.4 68.58) (end 149.86 68.58) (width 0.2) (layer "F.Cu") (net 15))
 (via (at 149.86 68.58) (size 0.6) (drill 0.3) (layers "F.Cu" "B.Cu") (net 15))
 (via (at 152.4 68.58) (size 0.6) (drill 0.3) (layers "F.Cu" "B.Cu") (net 15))
 (segment (start 152.4 68.58) (end 152.4 81.28) (width 0.2) (layer "B.Cu") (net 15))
 (segment (start 149.86 68.58) (end 149.86 60.96) (width 0.2) (layer "B.Cu") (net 15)))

